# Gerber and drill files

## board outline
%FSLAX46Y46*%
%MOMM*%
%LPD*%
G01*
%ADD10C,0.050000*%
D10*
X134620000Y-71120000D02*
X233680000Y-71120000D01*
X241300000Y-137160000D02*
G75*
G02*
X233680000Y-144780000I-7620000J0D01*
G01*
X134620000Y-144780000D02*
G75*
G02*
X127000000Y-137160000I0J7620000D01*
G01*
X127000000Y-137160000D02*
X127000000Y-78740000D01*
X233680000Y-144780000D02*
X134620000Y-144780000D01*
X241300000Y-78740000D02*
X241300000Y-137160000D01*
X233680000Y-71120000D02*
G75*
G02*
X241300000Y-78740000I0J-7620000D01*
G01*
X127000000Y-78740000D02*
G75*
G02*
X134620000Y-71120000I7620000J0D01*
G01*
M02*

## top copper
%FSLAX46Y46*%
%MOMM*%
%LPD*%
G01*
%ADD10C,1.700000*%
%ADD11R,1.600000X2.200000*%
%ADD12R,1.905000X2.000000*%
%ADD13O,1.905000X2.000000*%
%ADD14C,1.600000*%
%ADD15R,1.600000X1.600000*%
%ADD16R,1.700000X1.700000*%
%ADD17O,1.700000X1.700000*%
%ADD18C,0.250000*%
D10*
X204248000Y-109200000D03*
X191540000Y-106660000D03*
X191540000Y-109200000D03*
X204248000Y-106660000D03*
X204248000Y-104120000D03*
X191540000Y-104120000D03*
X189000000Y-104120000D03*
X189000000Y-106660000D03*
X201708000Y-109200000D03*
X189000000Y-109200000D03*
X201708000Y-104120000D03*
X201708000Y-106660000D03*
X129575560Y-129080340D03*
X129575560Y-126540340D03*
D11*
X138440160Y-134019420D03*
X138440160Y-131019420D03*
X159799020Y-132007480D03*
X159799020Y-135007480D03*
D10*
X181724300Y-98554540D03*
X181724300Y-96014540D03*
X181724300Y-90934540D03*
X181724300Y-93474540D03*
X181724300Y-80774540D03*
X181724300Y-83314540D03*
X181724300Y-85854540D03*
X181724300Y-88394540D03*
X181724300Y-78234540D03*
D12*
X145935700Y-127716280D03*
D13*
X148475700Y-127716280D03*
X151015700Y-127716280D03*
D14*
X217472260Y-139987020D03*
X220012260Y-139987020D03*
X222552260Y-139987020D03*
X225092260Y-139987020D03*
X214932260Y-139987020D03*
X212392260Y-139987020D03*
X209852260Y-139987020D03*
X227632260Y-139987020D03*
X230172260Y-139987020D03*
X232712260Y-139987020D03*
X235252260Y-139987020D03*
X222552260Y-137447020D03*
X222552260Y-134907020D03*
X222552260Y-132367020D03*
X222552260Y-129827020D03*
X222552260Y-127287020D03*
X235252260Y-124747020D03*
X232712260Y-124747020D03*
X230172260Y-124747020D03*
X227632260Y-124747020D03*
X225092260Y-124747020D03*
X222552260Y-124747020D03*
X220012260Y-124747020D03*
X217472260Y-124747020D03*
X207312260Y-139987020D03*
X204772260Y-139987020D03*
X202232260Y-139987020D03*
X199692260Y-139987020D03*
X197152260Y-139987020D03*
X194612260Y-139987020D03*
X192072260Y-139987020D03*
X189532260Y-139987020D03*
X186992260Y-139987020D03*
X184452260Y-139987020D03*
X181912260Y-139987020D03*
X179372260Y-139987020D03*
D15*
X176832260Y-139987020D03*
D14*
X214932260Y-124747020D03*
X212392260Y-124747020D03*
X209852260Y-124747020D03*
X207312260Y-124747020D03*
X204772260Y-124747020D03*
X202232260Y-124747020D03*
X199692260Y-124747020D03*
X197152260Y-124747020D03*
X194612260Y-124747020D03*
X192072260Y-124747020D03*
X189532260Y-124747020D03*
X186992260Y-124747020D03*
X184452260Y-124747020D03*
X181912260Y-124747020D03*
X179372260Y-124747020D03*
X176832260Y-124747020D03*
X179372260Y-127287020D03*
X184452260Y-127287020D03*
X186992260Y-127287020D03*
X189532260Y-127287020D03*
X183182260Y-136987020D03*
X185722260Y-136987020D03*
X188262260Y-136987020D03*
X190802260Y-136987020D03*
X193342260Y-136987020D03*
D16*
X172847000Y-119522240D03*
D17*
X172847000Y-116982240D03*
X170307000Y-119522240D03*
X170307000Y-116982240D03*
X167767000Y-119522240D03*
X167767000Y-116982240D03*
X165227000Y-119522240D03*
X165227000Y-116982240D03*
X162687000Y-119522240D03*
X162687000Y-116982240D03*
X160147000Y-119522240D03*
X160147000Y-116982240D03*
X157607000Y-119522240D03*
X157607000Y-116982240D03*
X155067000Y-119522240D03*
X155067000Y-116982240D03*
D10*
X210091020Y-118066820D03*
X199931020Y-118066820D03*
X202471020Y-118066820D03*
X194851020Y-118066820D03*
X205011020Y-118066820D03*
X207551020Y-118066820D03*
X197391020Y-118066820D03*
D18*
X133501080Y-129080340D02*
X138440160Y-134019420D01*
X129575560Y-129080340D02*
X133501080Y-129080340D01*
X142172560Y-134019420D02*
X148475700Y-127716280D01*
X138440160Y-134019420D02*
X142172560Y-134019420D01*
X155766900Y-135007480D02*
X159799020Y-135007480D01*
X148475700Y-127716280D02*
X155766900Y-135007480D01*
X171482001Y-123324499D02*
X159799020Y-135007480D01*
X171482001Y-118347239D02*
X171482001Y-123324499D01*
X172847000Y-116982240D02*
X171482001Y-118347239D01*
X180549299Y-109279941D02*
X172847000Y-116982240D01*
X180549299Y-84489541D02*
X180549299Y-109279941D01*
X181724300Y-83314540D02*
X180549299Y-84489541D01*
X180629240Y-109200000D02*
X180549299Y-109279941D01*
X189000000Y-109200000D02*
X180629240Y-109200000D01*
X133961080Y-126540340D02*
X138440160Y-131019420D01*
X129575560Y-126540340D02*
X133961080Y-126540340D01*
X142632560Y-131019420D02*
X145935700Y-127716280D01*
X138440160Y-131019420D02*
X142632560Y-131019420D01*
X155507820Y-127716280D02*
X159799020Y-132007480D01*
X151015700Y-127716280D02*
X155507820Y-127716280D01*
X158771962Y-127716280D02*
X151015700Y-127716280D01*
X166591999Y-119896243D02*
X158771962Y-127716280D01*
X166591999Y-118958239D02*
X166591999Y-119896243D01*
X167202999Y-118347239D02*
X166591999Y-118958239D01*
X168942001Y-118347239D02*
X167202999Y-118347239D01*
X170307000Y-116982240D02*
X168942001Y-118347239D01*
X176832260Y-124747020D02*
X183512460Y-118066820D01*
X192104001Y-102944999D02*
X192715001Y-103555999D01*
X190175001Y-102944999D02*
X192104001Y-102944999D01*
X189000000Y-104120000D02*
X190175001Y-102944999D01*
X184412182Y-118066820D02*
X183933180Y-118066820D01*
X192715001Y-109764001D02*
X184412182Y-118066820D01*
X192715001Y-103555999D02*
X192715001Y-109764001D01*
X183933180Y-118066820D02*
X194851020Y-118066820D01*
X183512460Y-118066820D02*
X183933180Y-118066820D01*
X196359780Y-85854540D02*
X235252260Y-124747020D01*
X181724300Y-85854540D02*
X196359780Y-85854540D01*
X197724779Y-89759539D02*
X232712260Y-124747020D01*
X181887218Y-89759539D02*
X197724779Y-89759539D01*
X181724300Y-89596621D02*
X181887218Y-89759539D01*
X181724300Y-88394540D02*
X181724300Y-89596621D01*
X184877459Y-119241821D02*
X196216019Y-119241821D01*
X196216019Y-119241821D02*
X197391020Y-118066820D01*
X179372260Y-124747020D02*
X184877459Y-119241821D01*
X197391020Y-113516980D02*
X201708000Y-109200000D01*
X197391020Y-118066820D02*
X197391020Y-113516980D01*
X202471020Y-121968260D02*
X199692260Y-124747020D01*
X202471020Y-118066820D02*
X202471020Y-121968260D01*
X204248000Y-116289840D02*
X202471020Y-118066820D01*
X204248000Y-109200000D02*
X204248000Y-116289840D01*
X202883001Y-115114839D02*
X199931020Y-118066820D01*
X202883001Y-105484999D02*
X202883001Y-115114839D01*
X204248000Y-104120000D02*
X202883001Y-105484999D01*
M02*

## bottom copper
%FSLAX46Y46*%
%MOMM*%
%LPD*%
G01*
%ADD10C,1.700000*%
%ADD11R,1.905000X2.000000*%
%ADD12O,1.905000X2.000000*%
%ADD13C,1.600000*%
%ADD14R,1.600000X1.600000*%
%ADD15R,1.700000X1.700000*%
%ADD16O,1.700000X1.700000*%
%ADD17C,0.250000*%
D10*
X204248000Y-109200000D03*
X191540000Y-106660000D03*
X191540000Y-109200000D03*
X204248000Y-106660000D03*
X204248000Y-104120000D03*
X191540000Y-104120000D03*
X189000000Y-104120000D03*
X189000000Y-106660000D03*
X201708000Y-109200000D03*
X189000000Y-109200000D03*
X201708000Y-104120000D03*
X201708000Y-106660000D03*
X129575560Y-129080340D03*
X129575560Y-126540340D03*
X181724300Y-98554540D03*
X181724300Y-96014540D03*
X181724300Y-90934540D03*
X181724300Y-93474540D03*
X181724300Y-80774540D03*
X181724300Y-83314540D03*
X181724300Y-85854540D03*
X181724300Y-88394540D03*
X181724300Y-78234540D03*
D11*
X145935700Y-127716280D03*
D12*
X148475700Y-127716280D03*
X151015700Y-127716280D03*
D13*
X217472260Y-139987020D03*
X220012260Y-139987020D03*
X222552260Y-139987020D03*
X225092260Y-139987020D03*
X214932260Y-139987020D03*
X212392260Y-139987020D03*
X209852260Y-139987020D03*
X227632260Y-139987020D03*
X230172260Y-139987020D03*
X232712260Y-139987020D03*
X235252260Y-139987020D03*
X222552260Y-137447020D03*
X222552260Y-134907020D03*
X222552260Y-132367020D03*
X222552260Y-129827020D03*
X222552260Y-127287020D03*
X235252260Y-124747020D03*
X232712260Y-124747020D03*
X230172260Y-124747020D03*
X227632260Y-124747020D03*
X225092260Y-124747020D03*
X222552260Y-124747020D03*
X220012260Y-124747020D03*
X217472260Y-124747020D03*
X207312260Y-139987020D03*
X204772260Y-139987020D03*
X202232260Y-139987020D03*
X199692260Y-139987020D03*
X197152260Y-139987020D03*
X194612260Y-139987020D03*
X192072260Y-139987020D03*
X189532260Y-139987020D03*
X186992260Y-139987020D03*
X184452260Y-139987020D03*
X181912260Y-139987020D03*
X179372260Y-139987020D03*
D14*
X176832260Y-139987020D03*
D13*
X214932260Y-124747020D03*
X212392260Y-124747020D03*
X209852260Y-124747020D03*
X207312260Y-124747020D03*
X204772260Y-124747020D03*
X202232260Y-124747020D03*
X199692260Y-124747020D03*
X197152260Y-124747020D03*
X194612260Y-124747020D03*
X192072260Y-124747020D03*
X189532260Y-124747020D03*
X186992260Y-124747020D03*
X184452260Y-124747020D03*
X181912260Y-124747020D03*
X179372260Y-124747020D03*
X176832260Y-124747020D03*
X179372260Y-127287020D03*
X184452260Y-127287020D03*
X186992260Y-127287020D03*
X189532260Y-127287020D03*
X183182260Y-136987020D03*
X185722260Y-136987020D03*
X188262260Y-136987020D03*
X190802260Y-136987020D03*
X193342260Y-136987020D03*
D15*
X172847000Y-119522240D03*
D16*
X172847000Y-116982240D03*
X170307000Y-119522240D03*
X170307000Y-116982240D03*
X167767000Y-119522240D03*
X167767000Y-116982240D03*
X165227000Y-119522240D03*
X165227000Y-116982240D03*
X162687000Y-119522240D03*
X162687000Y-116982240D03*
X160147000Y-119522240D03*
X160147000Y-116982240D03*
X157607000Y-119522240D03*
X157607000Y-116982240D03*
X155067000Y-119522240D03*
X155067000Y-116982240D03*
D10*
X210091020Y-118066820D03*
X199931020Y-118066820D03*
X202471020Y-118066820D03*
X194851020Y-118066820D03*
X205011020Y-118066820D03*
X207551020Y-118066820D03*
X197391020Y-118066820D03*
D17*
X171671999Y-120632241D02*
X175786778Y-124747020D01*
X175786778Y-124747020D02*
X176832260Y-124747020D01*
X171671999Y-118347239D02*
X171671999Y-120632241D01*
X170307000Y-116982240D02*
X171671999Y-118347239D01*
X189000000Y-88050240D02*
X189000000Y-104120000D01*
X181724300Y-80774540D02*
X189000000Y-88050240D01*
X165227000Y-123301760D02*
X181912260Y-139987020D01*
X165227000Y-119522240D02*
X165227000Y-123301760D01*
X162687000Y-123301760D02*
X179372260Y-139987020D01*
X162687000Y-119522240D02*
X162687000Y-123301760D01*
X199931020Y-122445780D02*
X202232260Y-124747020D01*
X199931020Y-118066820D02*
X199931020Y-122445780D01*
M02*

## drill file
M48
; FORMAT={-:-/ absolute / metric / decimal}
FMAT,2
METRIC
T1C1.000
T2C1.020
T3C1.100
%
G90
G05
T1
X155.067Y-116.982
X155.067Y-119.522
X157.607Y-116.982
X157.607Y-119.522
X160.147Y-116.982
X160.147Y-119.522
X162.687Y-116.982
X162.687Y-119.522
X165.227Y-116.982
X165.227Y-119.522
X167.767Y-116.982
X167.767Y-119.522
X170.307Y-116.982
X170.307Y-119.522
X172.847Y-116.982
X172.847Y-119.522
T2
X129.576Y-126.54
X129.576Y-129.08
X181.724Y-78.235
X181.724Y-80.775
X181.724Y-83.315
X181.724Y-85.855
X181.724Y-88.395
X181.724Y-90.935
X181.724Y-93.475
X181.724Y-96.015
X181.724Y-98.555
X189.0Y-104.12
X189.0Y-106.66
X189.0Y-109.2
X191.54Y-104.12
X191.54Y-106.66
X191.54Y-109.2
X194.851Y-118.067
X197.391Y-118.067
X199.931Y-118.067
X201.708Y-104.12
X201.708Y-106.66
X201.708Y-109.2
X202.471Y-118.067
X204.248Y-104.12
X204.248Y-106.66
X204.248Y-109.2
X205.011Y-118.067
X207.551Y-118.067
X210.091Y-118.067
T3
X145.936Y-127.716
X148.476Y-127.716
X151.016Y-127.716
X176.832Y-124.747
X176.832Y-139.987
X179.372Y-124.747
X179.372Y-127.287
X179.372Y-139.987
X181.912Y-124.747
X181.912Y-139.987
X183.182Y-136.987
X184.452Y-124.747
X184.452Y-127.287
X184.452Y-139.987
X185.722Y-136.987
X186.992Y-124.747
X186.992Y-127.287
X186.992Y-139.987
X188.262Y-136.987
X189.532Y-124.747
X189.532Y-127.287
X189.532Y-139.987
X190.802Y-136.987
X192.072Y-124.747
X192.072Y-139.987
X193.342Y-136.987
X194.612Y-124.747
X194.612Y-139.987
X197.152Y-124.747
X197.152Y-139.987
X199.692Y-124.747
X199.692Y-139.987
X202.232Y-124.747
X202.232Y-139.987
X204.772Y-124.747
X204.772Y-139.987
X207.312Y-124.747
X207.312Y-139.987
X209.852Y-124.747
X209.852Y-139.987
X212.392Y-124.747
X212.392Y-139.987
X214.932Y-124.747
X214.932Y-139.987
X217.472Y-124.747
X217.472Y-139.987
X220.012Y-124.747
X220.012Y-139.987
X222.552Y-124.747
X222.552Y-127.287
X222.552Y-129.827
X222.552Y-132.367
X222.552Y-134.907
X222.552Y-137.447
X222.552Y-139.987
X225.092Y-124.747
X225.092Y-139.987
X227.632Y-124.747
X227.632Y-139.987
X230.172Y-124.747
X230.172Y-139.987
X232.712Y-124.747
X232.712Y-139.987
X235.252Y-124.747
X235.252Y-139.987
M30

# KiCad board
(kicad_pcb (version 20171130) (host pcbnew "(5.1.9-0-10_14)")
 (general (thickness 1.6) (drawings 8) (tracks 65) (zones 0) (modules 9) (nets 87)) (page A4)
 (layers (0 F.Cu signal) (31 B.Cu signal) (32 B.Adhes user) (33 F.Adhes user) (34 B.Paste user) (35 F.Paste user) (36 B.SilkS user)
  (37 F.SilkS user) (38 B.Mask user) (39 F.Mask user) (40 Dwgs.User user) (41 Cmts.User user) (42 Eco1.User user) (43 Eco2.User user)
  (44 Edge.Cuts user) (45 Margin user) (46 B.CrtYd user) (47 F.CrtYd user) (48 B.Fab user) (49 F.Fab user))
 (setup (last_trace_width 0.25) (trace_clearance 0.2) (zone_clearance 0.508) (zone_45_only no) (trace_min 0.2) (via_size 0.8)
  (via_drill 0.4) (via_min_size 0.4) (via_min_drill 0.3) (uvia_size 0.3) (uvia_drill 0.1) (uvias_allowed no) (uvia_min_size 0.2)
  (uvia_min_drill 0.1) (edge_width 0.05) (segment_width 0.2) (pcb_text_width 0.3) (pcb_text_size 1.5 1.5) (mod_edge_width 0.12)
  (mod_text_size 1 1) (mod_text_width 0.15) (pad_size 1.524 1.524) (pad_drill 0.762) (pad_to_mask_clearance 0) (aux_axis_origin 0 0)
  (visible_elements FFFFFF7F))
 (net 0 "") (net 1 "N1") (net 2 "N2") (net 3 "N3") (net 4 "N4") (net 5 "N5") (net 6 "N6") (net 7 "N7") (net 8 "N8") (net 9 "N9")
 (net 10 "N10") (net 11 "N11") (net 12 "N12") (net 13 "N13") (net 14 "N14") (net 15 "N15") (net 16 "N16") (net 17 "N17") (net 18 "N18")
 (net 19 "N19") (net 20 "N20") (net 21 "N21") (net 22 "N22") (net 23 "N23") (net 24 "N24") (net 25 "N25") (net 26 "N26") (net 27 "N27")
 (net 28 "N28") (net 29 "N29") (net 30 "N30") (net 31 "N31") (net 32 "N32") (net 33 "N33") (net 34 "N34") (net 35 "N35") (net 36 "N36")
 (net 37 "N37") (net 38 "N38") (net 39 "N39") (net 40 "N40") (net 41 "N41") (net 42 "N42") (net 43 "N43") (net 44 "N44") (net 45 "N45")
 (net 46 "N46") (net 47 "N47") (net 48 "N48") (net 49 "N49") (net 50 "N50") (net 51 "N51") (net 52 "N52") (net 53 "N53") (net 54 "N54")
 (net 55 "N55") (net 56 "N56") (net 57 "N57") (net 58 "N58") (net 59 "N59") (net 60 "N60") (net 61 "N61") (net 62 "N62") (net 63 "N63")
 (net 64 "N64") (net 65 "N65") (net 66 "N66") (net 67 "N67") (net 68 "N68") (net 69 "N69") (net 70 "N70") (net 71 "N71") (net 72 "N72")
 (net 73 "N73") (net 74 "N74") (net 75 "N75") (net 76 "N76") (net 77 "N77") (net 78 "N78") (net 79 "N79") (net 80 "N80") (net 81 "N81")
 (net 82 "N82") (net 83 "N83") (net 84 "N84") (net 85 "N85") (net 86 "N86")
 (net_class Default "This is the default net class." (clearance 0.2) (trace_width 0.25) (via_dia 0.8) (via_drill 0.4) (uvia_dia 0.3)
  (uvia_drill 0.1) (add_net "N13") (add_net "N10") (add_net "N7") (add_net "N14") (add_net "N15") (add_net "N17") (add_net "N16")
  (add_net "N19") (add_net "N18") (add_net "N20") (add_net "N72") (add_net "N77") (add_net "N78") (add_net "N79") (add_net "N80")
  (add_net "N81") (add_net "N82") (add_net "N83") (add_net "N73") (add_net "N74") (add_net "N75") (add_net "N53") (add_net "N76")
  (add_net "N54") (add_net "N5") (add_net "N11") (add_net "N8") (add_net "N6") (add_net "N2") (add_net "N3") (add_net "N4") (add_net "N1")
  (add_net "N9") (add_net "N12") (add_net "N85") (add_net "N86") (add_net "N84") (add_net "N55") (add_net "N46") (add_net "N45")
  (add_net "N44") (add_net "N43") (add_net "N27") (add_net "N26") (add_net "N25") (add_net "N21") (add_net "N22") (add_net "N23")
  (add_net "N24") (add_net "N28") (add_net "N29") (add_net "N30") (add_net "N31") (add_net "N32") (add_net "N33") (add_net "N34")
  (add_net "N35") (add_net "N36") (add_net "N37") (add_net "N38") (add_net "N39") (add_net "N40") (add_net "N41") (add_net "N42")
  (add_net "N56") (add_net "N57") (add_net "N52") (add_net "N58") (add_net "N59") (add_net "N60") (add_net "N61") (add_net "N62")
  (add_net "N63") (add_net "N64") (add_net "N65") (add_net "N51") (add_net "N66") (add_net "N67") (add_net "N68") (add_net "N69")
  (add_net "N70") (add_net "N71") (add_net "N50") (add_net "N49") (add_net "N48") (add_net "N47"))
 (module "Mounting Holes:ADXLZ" (layer F.Cu) (at 189 109.2)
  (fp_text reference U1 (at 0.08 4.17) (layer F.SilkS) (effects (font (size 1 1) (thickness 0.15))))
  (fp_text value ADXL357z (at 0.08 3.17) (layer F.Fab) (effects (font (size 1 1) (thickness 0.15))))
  (pad 3 thru_hole circle (at 15.248 0) (size 1.7 1.7) (drill 1.02) (layers *.Cu *.Mask) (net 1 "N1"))
  (pad 13 thru_hole circle (at 2.54 -2.54) (size 1.7 1.7) (drill 1.02) (layers *.Cu *.Mask) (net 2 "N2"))
  (pad 14 thru_hole circle (at 2.54 0) (size 1.7 1.7) (drill 1.02) (layers *.Cu *.Mask) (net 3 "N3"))
  (pad 2 thru_hole circle (at 15.248 -2.54) (size 1.7 1.7) (drill 1.02) (layers *.Cu *.Mask) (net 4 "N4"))
  (pad 1 thru_hole circle (at 15.248 -5.08) (size 1.7 1.7) (drill 1.02) (layers *.Cu *.Mask) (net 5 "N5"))
  (pad 12 thru_hole circle (at 2.54 -5.08) (size 1.7 1.7) (drill 1.02) (layers *.Cu *.Mask) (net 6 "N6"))
  (pad 5 thru_hole circle (at 0 -5.08) (size 1.7 1.7) (drill 1.02) (layers *.Cu *.Mask) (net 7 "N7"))
  (pad 11 thru_hole circle (at 0 -2.54) (size 1.7 1.7) (drill 1.02) (layers *.Cu *.Mask) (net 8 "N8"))
  (pad 4 thru_hole circle (at 12.708 0) (size 1.7 1.7) (drill 1.02) (layers *.Cu *.Mask) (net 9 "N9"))
  (pad 6 thru_hole circle (at 0 0) (size 1.7 1.7) (drill 1.02) (layers *.Cu *.Mask) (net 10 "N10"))
  (pad 10 thru_hole circle (at 12.708 -5.08) (size 1.7 1.7) (drill 1.02) (layers *.Cu *.Mask) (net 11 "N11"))
  (pad 8 thru_hole circle (at 12.708 -2.54) (size 1.7 1.7) (drill 1.02) (layers *.Cu *.Mask) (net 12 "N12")))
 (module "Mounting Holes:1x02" (layer F.Cu) (at 129.57556 123.37034 180)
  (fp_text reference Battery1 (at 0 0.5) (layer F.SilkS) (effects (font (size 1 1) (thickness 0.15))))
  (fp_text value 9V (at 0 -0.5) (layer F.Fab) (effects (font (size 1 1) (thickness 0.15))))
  (pad 2 thru_hole circle (at 0 -5.71 180) (size 1.7 1.7) (drill 1.02) (layers *.Cu *.Mask) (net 10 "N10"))
  (pad 1 thru_hole circle (at 0 -3.17 180) (size 1.7 1.7) (drill 1.02) (layers *.Cu *.Mask) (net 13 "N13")))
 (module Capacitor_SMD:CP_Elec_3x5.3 (layer F.Cu) (at 138.44016 132.51942 270)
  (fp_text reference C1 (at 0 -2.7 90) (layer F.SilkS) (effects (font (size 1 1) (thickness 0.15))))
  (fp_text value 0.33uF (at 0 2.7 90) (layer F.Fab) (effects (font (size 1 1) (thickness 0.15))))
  (pad 2 smd rect (at 1.5 0 270) (size 2.2 1.6) (layers F.Cu F.Paste F.Mask) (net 10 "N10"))
  (pad 1 smd rect (at -1.5 0 270) (size 2.2 1.6) (layers F.Cu F.Paste F.Mask) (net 13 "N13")))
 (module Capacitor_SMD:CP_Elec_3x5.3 (layer F.Cu) (at 159.79902 133.50748 270)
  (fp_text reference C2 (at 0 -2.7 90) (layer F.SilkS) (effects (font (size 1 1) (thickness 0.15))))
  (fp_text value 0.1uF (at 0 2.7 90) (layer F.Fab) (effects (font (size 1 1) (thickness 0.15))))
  (pad 1 smd rect (at -1.5 0 270) (size 2.2 1.6) (layers F.Cu F.Paste F.Mask) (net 7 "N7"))
  (pad 2 smd rect (at 1.5 0 270) (size 2.2 1.6) (layers F.Cu F.Paste F.Mask) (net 10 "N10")))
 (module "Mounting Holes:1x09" (layer F.Cu) (at 181.7243 98.55454)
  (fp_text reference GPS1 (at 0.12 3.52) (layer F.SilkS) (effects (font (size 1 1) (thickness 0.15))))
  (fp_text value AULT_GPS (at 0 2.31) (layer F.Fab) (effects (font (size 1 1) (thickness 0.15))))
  (pad 1 thru_hole circle (at 0 0) (size 1.7 1.7) (drill 1.02) (layers *.Cu *.Mask) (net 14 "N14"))
  (pad 2 thru_hole circle (at 0 -2.54) (size 1.7 1.7) (drill 1.02) (layers *.Cu *.Mask) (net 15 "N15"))
  (pad 4 thru_hole circle (at 0 -7.62) (size 1.7 1.7) (drill 1.02) (layers *.Cu *.Mask) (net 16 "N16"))
  (pad 3 thru_hole circle (at 0 -5.08) (size 1.7 1.7) (drill 1.02) (layers *.Cu *.Mask) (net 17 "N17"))
  (pad 8 thru_hole circle (at 0 -17.78) (size 1.7 1.7) (drill 1.02) (layers *.Cu *.Mask) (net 7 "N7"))
  (pad 7 thru_hole circle (at 0 -15.24) (size 1.7 1.7) (drill 1.02) (layers *.Cu *.Mask) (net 10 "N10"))
  (pad 6 thru_hole circle (at 0 -12.7) (size 1.7 1.7) (drill 1.02) (layers *.Cu *.Mask) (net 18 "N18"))
  (pad 5 thru_hole circle (at 0 -10.16) (size 1.7 1.7) (drill 1.02) (layers *.Cu *.Mask) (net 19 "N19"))
  (pad 9 thru_hole circle (at 0 -20.32) (size 1.7 1.7) (drill 1.02) (layers *.Cu *.Mask) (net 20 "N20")))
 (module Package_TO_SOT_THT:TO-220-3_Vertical (layer F.Cu) (at 145.9357 127.71628)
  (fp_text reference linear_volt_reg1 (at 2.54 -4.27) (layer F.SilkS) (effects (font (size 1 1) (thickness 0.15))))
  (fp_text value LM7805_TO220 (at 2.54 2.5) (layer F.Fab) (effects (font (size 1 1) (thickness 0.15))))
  (pad 1 thru_hole rect (at 0 0) (size 1.905 2) (drill 1.1) (layers *.Cu *.Mask) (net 13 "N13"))
  (pad 2 thru_hole oval (at 2.54 0) (size 1.905 2) (drill 1.1) (layers *.Cu *.Mask) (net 10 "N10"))
  (pad 3 thru_hole oval (at 5.08 0) (size 1.905 2) (drill 1.1) (layers *.Cu *.Mask) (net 7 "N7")))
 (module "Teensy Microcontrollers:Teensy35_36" (layer F.Cu) (at 206.04226 132.36702)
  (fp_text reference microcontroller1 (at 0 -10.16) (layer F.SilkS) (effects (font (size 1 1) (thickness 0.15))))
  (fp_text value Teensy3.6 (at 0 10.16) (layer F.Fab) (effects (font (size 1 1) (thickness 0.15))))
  (pad 17 thru_hole circle (at 11.43 7.62) (size 1.6 1.6) (drill 1.1) (layers *.Cu *.Mask) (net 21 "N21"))
  (pad 18 thru_hole circle (at 13.97 7.62) (size 1.6 1.6) (drill 1.1) (layers *.Cu *.Mask) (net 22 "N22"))
  (pad 19 thru_hole circle (at 16.51 7.62) (size 1.6 1.6) (drill 1.1) (layers *.Cu *.Mask) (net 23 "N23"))
  (pad 20 thru_hole circle (at 19.05 7.62) (size 1.6 1.6) (drill 1.1) (layers *.Cu *.Mask) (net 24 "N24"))
  (pad 16 thru_hole circle (at 8.89 7.62) (size 1.6 1.6) (drill 1.1) (layers *.Cu *.Mask) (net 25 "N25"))
  (pad 15 thru_hole circle (at 6.35 7.62) (size 1.6 1.6) (drill 1.1) (layers *.Cu *.Mask) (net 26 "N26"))
  (pad 14 thru_hole circle (at 3.81 7.62) (size 1.6 1.6) (drill 1.1) (layers *.Cu *.Mask) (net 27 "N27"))
  (pad 21 thru_hole circle (at 21.59 7.62) (size 1.6 1.6) (drill 1.1) (layers *.Cu *.Mask) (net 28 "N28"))
  (pad 22 thru_hole circle (at 24.13 7.62) (size 1.6 1.6) (drill 1.1) (layers *.Cu *.Mask) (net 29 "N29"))
  (pad 23 thru_hole circle (at 26.67 7.62) (size 1.6 1.6) (drill 1.1) (layers *.Cu *.Mask) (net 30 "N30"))
  (pad 24 thru_hole circle (at 29.21 7.62) (size 1.6 1.6) (drill 1.1) (layers *.Cu *.Mask) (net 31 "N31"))
  (pad 25 thru_hole circle (at 16.51 5.08) (size 1.6 1.6) (drill 1.1) (layers *.Cu *.Mask) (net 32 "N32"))
  (pad 26 thru_hole circle (at 16.51 2.54) (size 1.6 1.6) (drill 1.1) (layers *.Cu *.Mask) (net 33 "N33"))
  (pad 27 thru_hole circle (at 16.51 0) (size 1.6 1.6) (drill 1.1) (layers *.Cu *.Mask) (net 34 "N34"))
  (pad 28 thru_hole circle (at 16.51 -2.54) (size 1.6 1.6) (drill 1.1) (layers *.Cu *.Mask) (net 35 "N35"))
  (pad 29 thru_hole circle (at 16.51 -5.08) (size 1.6 1.6) (drill 1.1) (layers *.Cu *.Mask) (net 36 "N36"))
  (pad 30 thru_hole circle (at 29.21 -7.62) (size 1.6 1.6) (drill 1.1) (layers *.Cu *.Mask) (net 18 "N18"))
  (pad 31 thru_hole circle (at 26.67 -7.62) (size 1.6 1.6) (drill 1.1) (layers *.Cu *.Mask) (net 19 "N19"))
  (pad 32 thru_hole circle (at 24.13 -7.62) (size 1.6 1.6) (drill 1.1) (layers *.Cu *.Mask) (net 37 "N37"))
  (pad 33 thru_hole circle (at 21.59 -7.62) (size 1.6 1.6) (drill 1.1) (layers *.Cu *.Mask) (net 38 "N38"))
  (pad 34 thru_hole circle (at 19.05 -7.62) (size 1.6 1.6) (drill 1.1) (layers *.Cu *.Mask) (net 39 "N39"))
  (pad 35 thru_hole circle (at 16.51 -7.62) (size 1.6 1.6) (drill 1.1) (layers *.Cu *.Mask) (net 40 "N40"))
  (pad 36 thru_hole circle (at 13.97 -7.62) (size 1.6 1.6) (drill 1.1) (layers *.Cu *.Mask) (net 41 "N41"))
  (pad 37 thru_hole circle (at 11.43 -7.62) (size 1.6 1.6) (drill 1.1) (layers *.Cu *.Mask) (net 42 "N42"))
  (pad 13 thru_hole circle (at 1.27 7.62) (size 1.6 1.6) (drill 1.1) (layers *.Cu *.Mask) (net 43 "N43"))
  (pad 12 thru_hole circle (at -1.27 7.62) (size 1.6 1.6) (drill 1.1) (layers *.Cu *.Mask) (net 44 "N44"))
  (pad 11 thru_hole circle (at -3.81 7.62) (size 1.6 1.6) (drill 1.1) (layers *.Cu *.Mask) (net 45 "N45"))
  (pad 10 thru_hole circle (at -6.35 7.62) (size 1.6 1.6) (drill 1.1) (layers *.Cu *.Mask) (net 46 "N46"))
  (pad 9 thru_hole circle (at -8.89 7.62) (size 1.6 1.6) (drill 1.1) (layers *.Cu *.Mask) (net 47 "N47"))
  (pad 8 thru_hole circle (at -11.43 7.62) (size 1.6 1.6) (drill 1.1) (layers *.Cu *.Mask) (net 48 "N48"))
  (pad 7 thru_hole circle (at -13.97 7.62) (size 1.6 1.6) (drill 1.1) (layers *.Cu *.Mask) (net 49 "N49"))
  (pad 6 thru_hole circle (at -16.51 7.62) (size 1.6 1.6) (drill 1.1) (layers *.Cu *.Mask) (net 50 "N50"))
  (pad 5 thru_hole circle (at -19.05 7.62) (size 1.6 1.6) (drill 1.1) (layers *.Cu *.Mask) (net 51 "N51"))
  (pad 4 thru_hole circle (at -21.59 7.62) (size 1.6 1.6) (drill 1.1) (layers *.Cu *.Mask) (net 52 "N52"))
  (pad 3 thru_hole circle (at -24.13 7.62) (size 1.6 1.6) (drill 1.1) (layers *.Cu *.Mask) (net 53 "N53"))
  (pad 2 thru_hole circle (at -26.67 7.62) (size 1.6 1.6) (drill 1.1) (layers *.Cu *.Mask) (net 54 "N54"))
  (pad 1 thru_hole rect (at -29.21 7.62) (size 1.6 1.6) (drill 1.1) (layers *.Cu *.Mask) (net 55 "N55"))
  (pad 38 thru_hole circle (at 8.89 -7.62) (size 1.6 1.6) (drill 1.1) (layers *.Cu *.Mask) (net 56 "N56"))
  (pad 39 thru_hole circle (at 6.35 -7.62) (size 1.6 1.6) (drill 1.1) (layers *.Cu *.Mask) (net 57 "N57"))
  (pad 40 thru_hole circle (at 3.81 -7.62) (size 1.6 1.6) (drill 1.1) (layers *.Cu *.Mask) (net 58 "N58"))
  (pad 41 thru_hole circle (at 1.27 -7.62) (size 1.6 1.6) (drill 1.1) (layers *.Cu *.Mask) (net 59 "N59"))
  (pad 42 thru_hole circle (at -1.27 -7.62) (size 1.6 1.6) (drill 1.1) (layers *.Cu *.Mask) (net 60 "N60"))
  (pad 43 thru_hole circle (at -3.81 -7.62) (size 1.6 1.6) (drill 1.1) (layers *.Cu *.Mask) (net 5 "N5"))
  (pad 44 thru_hole circle (at -6.35 -7.62) (size 1.6 1.6) (drill 1.1) (layers *.Cu *.Mask) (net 1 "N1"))
  (pad 45 thru_hole circle (at -8.89 -7.62) (size 1.6 1.6) (drill 1.1) (layers *.Cu *.Mask) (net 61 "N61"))
  (pad 46 thru_hole circle (at -11.43 -7.62) (size 1.6 1.6) (drill 1.1) (layers *.Cu *.Mask) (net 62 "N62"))
  (pad 47 thru_hole circle (at -13.97 -7.62) (size 1.6 1.6) (drill 1.1) (layers *.Cu *.Mask) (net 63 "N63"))
  (pad 48 thru_hole circle (at -16.51 -7.62) (size 1.6 1.6) (drill 1.1) (layers *.Cu *.Mask) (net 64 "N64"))
  (pad 49 thru_hole circle (at -19.05 -7.62) (size 1.6 1.6) (drill 1.1) (layers *.Cu *.Mask) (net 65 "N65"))
  (pad 50 thru_hole circle (at -21.59 -7.62) (size 1.6 1.6) (drill 1.1) (layers *.Cu *.Mask) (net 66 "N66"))
  (pad 51 thru_hole circle (at -24.13 -7.62) (size 1.6 1.6) (drill 1.1) (layers *.Cu *.Mask) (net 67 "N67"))
  (pad 52 thru_hole circle (at -26.67 -7.62) (size 1.6 1.6) (drill 1.1) (layers *.Cu *.Mask) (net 9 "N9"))
  (pad 53 thru_hole circle (at -29.21 -7.62) (size 1.6 1.6) (drill 1.1) (layers *.Cu *.Mask) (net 7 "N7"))
  (pad 54 thru_hole circle (at -26.67 -5.08) (size 1.6 1.6) (drill 1.1) (layers *.Cu *.Mask) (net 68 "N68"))
  (pad 55 thru_hole circle (at -21.59 -5.08) (size 1.6 1.6) (drill 1.1) (layers *.Cu *.Mask) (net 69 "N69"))
  (pad 56 thru_hole circle (at -19.05 -5.08) (size 1.6 1.6) (drill 1.1) (layers *.Cu *.Mask) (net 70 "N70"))
  (pad 57 thru_hole circle (at -16.51 -5.08) (size 1.6 1.6) (drill 1.1) (layers *.Cu *.Mask) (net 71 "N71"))
  (pad 58 thru_hole circle (at -22.86 4.62) (size 1.6 1.6) (drill 1.1) (layers *.Cu *.Mask))
  (pad 59 thru_hole circle (at -20.32 4.62) (size 1.6 1.6) (drill 1.1) (layers *.Cu *.Mask))
  (pad 60 thru_hole circle (at -17.78 4.62) (size 1.6 1.6) (drill 1.1) (layers *.Cu *.Mask))
  (pad 61 thru_hole circle (at -15.24 4.62) (size 1.6 1.6) (drill 1.1) (layers *.Cu *.Mask))
  (pad 62 thru_hole circle (at -12.7 4.62) (size 1.6 1.6) (drill 1.1) (layers *.Cu *.Mask)))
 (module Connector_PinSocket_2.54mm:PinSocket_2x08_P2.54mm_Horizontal (layer F.Cu) (at 172.847 119.52224 270)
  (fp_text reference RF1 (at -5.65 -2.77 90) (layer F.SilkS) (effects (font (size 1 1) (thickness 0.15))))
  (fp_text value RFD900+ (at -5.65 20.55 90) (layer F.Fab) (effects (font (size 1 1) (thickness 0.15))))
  (pad 1 thru_hole rect (at 0 0 270) (size 1.7 1.7) (drill 1) (layers *.Cu *.Mask) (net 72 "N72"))
  (pad 2 thru_hole oval (at -2.54 0 270) (size 1.7 1.7) (drill 1) (layers *.Cu *.Mask) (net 10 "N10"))
  (pad 3 thru_hole oval (at 0 2.54 270) (size 1.7 1.7) (drill 1) (layers *.Cu *.Mask) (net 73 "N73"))
  (pad 4 thru_hole oval (at -2.54 2.54 270) (size 1.7 1.7) (drill 1) (layers *.Cu *.Mask) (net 7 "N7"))
  (pad 5 thru_hole oval (at 0 5.08 270) (size 1.7 1.7) (drill 1) (layers *.Cu *.Mask) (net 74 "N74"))
  (pad 6 thru_hole oval (at -2.54 5.08 270) (size 1.7 1.7) (drill 1) (layers *.Cu *.Mask) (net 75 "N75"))
  (pad 7 thru_hole oval (at 0 7.62 270) (size 1.7 1.7) (drill 1) (layers *.Cu *.Mask) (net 53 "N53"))
  (pad 8 thru_hole oval (at -2.54 7.62 270) (size 1.7 1.7) (drill 1) (layers *.Cu *.Mask) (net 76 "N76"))
  (pad 9 thru_hole oval (at 0 10.16 270) (size 1.7 1.7) (drill 1) (layers *.Cu *.Mask) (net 54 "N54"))
  (pad 10 thru_hole oval (at -2.54 10.16 270) (size 1.7 1.7) (drill 1) (layers *.Cu *.Mask) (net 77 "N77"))
  (pad 11 thru_hole oval (at 0 12.7 270) (size 1.7 1.7) (drill 1) (layers *.Cu *.Mask) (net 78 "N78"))
  (pad 12 thru_hole oval (at -2.54 12.7 270) (size 1.7 1.7) (drill 1) (layers *.Cu *.Mask) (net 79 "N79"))
  (pad 13 thru_hole oval (at 0 15.24 270) (size 1.7 1.7) (drill 1) (layers *.Cu *.Mask) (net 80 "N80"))
  (pad 14 thru_hole oval (at -2.54 15.24 270) (size 1.7 1.7) (drill 1) (layers *.Cu *.Mask) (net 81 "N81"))
  (pad 15 thru_hole oval (at 0 17.78 270) (size 1.7 1.7) (drill 1) (layers *.Cu *.Mask) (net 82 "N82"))
  (pad 16 thru_hole oval (at -2.54 17.78 270) (size 1.7 1.7) (drill 1) (layers *.Cu *.Mask) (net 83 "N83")))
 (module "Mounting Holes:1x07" (layer F.Cu) (at 192.53102 118.08682 270)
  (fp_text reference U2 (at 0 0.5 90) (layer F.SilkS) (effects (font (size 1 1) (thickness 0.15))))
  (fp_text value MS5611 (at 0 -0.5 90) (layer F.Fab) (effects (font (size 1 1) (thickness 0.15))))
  (pad 7 thru_hole circle (at -0.02 -17.56 270) (size 1.7 1.7) (drill 1.02) (layers *.Cu *.Mask) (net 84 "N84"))
  (pad 3 thru_hole circle (at -0.02 -7.4 270) (size 1.7 1.7) (drill 1.02) (layers *.Cu *.Mask) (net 5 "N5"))
  (pad 4 thru_hole circle (at -0.02 -9.94 270) (size 1.7 1.7) (drill 1.02) (layers *.Cu *.Mask) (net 1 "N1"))
  (pad 1 thru_hole circle (at -0.02 -2.32 270) (size 1.7 1.7) (drill 1.02) (layers *.Cu *.Mask) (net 7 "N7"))
  (pad 5 thru_hole circle (at -0.02 -12.48 270) (size 1.7 1.7) (drill 1.02) (layers *.Cu *.Mask) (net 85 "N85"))
  (pad 6 thru_hole circle (at -0.02 -15.02 270) (size 1.7 1.7) (drill 1.02) (layers *.Cu *.Mask) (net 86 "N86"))
  (pad 2 thru_hole circle (at -0.02 -4.86 270) (size 1.7 1.7) (drill 1.02) (layers *.Cu *.Mask) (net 9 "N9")))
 (gr_line (start 134.62 71.12) (end 233.68 71.12) (layer Edge.Cuts) (width 0.05))
 (gr_arc (start 233.68 137.16) (end 233.68 144.78) (angle -90) (layer Edge.Cuts) (width 0.05))
 (gr_arc (start 134.62 137.16) (end 127 137.16) (angle -90) (layer Edge.Cuts) (width 0.05))
 (gr_line (start 127 137.16) (end 127 78.74) (layer Edge.Cuts) (width 0.05))
 (gr_line (start 233.68 144.78) (end 134.62 144.78) (layer Edge.Cuts) (width 0.05))
 (gr_line (start 241.3 78.74) (end 241.3 137.16) (layer Edge.Cuts) (width 0.05))
 (gr_arc (start 233.68 78.74) (end 241.3 78.74) (angle -90) (layer Edge.Cuts) (width 0.05))
 (gr_arc (start 134.62 78.74) (end 134.62 71.12) (angle -90) (layer Edge.Cuts) (width 0.05))
 (segment (start 133.50108 129.08034) (end 138.44016 134.01942) (width 0.25) (layer F.Cu) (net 10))
 (segment (start 129.57556 129.08034) (end 133.50108 129.08034) (width 0.25) (layer F.Cu) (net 10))
 (segment (start 142.17256 134.01942) (end 148.4757 127.71628) (width 0.25) (layer F.Cu) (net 10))
 (segment (start 138.44016 134.01942) (end 142.17256 134.01942) (width 0.25) (layer F.Cu) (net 10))
 (segment (start 155.7669 135.00748) (end 159.79902 135.00748) (width 0.25) (layer F.Cu) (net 10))
 (segment (start 148.4757 127.71628) (end 155.7669 135.00748) (width 0.25) (layer F.Cu) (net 10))
 (segment (start 171.482001 123.324499) (end 159.79902 135.00748) (width 0.25) (layer F.Cu) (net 10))
 (segment (start 171.482001 118.347239) (end 171.482001 123.324499) (width 0.25) (layer F.Cu) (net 10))
 (segment (start 172.847 116.98224) (end 171.482001 118.347239) (width 0.25) (layer F.Cu) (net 10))
 (segment (start 180.549299 109.279941) (end 172.847 116.98224) (width 0.25) (layer F.Cu) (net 10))
 (segment (start 180.549299 84.489541) (end 180.549299 109.279941) (width 0.25) (layer F.Cu) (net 10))
 (segment (start 181.7243 83.31454) (end 180.549299 84.489541) (width 0.25) (layer F.Cu) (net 10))
 (segment (start 180.62924 109.2) (end 180.549299 109.279941) (width 0.25) (layer F.Cu) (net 10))
 (segment (start 189 109.2) (end 180.62924 109.2) (width 0.25) (layer F.Cu) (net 10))
 (segment (start 133.96108 126.54034) (end 138.44016 131.01942) (width 0.25) (layer F.Cu) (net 13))
 (segment (start 129.57556 126.54034) (end 133.96108 126.54034) (width 0.25) (layer F.Cu) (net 13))
 (segment (start 142.63256 131.01942) (end 145.9357 127.71628) (width 0.25) (layer F.Cu) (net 13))
 (segment (start 138.44016 131.01942) (end 142.63256 131.01942) (width 0.25) (layer F.Cu) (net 13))
 (segment (start 155.50782 127.71628) (end 159.79902 132.00748) (width 0.25) (layer F.Cu) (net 7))
 (segment (start 151.0157 127.71628) (end 155.50782 127.71628) (width 0.25) (layer F.Cu) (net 7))
 (segment (start 158.771962 127.71628) (end 151.0157 127.71628) (width 0.25) (layer F.Cu) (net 7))
 (segment (start 166.591999 119.896243) (end 158.771962 127.71628) (width 0.25) (layer F.Cu) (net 7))
 (segment (start 166.591999 118.958239) (end 166.591999 119.896243) (width 0.25) (layer F.Cu) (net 7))
 (segment (start 167.202999 118.347239) (end 166.591999 118.958239) (width 0.25) (layer F.Cu) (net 7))
 (segment (start 168.942001 118.347239) (end 167.202999 118.347239) (width 0.25) (layer F.Cu) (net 7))
 (segment (start 170.307 116.98224) (end 168.942001 118.347239) (width 0.25) (layer F.Cu) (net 7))
 (segment (start 171.671999 120.632241) (end 175.786778 124.74702) (width 0.25) (layer B.Cu) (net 7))
 (segment (start 175.786778 124.74702) (end 176.83226 124.74702) (width 0.25) (layer B.Cu) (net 7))
 (segment (start 171.671999 118.347239) (end 171.671999 120.632241) (width 0.25) (layer B.Cu) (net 7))
 (segment (start 170.307 116.98224) (end 171.671999 118.347239) (width 0.25) (layer B.Cu) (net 7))
 (segment (start 176.83226 124.74702) (end 183.51246 118.06682) (width 0.25) (layer F.Cu) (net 7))
 (segment (start 192.104001 102.944999) (end 192.715001 103.555999) (width 0.25) (layer F.Cu) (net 7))
 (segment (start 190.175001 102.944999) (end 192.104001 102.944999) (width 0.25) (layer F.Cu) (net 7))
 (segment (start 189 104.12) (end 190.175001 102.944999) (width 0.25) (layer F.Cu) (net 7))
 (segment (start 184.412182 118.06682) (end 183.93318 118.06682) (width 0.25) (layer F.Cu) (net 7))
 (segment (start 192.715001 109.764001) (end 184.412182 118.06682) (width 0.25) (layer F.Cu) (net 7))
 (segment (start 192.715001 103.555999) (end 192.715001 109.764001) (width 0.25) (layer F.Cu) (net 7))
 (segment (start 183.93318 118.06682) (end 194.85102 118.06682) (width 0.25) (layer F.Cu) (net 7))
 (segment (start 183.51246 118.06682) (end 183.93318 118.06682) (width 0.25) (layer F.Cu) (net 7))
 (segment (start 189 88.05024) (end 189 104.12) (width 0.25) (layer B.Cu) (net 7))
 (segment (start 181.7243 80.77454) (end 189 88.05024) (width 0.25) (layer B.Cu) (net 7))
 (segment (start 196.35978 85.85454) (end 235.25226 124.74702) (width 0.25) (layer F.Cu) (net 18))
 (segment (start 181.7243 85.85454) (end 196.35978 85.85454) (width 0.25) (layer F.Cu) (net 18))
 (segment (start 197.724779 89.759539) (end 232.71226 124.74702) (width 0.25) (layer F.Cu) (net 19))
 (segment (start 181.887218 89.759539) (end 197.724779 89.759539) (width 0.25) (layer F.Cu) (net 19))
 (segment (start 181.7243 89.596621) (end 181.887218 89.759539) (width 0.25) (layer F.Cu) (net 19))
 (segment (start 181.7243 88.39454) (end 181.7243 89.596621) (width 0.25) (layer F.Cu) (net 19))
 (segment (start 184.877459 119.241821) (end 196.216019 119.241821) (width 0.25) (layer F.Cu) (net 9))
 (segment (start 196.216019 119.241821) (end 197.39102 118.06682) (width 0.25) (layer F.Cu) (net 9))
 (segment (start 179.37226 124.74702) (end 184.877459 119.241821) (width 0.25) (layer F.Cu) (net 9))
 (segment (start 197.39102 113.51698) (end 201.708 109.2) (width 0.25) (layer F.Cu) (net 9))
 (segment (start 197.39102 118.06682) (end 197.39102 113.51698) (width 0.25) (layer F.Cu) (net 9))
 (segment (start 165.227 123.30176) (end 181.91226 139.98702) (width 0.25) (layer B.Cu) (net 53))
 (segment (start 165.227 119.52224) (end 165.227 123.30176) (width 0.25) (layer B.Cu) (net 53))
 (segment (start 162.687 123.30176) (end 179.37226 139.98702) (width 0.25) (layer B.Cu) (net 54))
 (segment (start 162.687 119.52224) (end 162.687 123.30176) (width 0.25) (layer B.Cu) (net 54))
 (segment (start 199.93102 122.44578) (end 202.23226 124.74702) (width 0.25) (layer B.Cu) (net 5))
 (segment (start 199.93102 118.06682) (end 199.93102 122.44578) (width 0.25) (layer B.Cu) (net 5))
 (segment (start 202.47102 121.96826) (end 199.69226 124.74702) (width 0.25) (layer F.Cu) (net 1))
 (segment (start 202.47102 118.06682) (end 202.47102 121.96826) (width 0.25) (layer F.Cu) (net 1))
 (segment (start 204.248 116.28984) (end 202.47102 118.06682) (width 0.25) (layer F.Cu) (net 1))
 (segment (start 204.248 109.2) (end 204.248 116.28984) (width 0.25) (layer F.Cu) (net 1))
 (segment (start 202.883001 115.114839) (end 199.93102 118.06682) (width 0.25) (layer F.Cu) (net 5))
 (segment (start 202.883001 105.484999) (end 202.883001 115.114839) (width 0.25) (layer F.Cu) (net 5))
 (segment (start 204.248 104.12) (end 202.883001 105.484999) (width 0.25) (layer F.Cu) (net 5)))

